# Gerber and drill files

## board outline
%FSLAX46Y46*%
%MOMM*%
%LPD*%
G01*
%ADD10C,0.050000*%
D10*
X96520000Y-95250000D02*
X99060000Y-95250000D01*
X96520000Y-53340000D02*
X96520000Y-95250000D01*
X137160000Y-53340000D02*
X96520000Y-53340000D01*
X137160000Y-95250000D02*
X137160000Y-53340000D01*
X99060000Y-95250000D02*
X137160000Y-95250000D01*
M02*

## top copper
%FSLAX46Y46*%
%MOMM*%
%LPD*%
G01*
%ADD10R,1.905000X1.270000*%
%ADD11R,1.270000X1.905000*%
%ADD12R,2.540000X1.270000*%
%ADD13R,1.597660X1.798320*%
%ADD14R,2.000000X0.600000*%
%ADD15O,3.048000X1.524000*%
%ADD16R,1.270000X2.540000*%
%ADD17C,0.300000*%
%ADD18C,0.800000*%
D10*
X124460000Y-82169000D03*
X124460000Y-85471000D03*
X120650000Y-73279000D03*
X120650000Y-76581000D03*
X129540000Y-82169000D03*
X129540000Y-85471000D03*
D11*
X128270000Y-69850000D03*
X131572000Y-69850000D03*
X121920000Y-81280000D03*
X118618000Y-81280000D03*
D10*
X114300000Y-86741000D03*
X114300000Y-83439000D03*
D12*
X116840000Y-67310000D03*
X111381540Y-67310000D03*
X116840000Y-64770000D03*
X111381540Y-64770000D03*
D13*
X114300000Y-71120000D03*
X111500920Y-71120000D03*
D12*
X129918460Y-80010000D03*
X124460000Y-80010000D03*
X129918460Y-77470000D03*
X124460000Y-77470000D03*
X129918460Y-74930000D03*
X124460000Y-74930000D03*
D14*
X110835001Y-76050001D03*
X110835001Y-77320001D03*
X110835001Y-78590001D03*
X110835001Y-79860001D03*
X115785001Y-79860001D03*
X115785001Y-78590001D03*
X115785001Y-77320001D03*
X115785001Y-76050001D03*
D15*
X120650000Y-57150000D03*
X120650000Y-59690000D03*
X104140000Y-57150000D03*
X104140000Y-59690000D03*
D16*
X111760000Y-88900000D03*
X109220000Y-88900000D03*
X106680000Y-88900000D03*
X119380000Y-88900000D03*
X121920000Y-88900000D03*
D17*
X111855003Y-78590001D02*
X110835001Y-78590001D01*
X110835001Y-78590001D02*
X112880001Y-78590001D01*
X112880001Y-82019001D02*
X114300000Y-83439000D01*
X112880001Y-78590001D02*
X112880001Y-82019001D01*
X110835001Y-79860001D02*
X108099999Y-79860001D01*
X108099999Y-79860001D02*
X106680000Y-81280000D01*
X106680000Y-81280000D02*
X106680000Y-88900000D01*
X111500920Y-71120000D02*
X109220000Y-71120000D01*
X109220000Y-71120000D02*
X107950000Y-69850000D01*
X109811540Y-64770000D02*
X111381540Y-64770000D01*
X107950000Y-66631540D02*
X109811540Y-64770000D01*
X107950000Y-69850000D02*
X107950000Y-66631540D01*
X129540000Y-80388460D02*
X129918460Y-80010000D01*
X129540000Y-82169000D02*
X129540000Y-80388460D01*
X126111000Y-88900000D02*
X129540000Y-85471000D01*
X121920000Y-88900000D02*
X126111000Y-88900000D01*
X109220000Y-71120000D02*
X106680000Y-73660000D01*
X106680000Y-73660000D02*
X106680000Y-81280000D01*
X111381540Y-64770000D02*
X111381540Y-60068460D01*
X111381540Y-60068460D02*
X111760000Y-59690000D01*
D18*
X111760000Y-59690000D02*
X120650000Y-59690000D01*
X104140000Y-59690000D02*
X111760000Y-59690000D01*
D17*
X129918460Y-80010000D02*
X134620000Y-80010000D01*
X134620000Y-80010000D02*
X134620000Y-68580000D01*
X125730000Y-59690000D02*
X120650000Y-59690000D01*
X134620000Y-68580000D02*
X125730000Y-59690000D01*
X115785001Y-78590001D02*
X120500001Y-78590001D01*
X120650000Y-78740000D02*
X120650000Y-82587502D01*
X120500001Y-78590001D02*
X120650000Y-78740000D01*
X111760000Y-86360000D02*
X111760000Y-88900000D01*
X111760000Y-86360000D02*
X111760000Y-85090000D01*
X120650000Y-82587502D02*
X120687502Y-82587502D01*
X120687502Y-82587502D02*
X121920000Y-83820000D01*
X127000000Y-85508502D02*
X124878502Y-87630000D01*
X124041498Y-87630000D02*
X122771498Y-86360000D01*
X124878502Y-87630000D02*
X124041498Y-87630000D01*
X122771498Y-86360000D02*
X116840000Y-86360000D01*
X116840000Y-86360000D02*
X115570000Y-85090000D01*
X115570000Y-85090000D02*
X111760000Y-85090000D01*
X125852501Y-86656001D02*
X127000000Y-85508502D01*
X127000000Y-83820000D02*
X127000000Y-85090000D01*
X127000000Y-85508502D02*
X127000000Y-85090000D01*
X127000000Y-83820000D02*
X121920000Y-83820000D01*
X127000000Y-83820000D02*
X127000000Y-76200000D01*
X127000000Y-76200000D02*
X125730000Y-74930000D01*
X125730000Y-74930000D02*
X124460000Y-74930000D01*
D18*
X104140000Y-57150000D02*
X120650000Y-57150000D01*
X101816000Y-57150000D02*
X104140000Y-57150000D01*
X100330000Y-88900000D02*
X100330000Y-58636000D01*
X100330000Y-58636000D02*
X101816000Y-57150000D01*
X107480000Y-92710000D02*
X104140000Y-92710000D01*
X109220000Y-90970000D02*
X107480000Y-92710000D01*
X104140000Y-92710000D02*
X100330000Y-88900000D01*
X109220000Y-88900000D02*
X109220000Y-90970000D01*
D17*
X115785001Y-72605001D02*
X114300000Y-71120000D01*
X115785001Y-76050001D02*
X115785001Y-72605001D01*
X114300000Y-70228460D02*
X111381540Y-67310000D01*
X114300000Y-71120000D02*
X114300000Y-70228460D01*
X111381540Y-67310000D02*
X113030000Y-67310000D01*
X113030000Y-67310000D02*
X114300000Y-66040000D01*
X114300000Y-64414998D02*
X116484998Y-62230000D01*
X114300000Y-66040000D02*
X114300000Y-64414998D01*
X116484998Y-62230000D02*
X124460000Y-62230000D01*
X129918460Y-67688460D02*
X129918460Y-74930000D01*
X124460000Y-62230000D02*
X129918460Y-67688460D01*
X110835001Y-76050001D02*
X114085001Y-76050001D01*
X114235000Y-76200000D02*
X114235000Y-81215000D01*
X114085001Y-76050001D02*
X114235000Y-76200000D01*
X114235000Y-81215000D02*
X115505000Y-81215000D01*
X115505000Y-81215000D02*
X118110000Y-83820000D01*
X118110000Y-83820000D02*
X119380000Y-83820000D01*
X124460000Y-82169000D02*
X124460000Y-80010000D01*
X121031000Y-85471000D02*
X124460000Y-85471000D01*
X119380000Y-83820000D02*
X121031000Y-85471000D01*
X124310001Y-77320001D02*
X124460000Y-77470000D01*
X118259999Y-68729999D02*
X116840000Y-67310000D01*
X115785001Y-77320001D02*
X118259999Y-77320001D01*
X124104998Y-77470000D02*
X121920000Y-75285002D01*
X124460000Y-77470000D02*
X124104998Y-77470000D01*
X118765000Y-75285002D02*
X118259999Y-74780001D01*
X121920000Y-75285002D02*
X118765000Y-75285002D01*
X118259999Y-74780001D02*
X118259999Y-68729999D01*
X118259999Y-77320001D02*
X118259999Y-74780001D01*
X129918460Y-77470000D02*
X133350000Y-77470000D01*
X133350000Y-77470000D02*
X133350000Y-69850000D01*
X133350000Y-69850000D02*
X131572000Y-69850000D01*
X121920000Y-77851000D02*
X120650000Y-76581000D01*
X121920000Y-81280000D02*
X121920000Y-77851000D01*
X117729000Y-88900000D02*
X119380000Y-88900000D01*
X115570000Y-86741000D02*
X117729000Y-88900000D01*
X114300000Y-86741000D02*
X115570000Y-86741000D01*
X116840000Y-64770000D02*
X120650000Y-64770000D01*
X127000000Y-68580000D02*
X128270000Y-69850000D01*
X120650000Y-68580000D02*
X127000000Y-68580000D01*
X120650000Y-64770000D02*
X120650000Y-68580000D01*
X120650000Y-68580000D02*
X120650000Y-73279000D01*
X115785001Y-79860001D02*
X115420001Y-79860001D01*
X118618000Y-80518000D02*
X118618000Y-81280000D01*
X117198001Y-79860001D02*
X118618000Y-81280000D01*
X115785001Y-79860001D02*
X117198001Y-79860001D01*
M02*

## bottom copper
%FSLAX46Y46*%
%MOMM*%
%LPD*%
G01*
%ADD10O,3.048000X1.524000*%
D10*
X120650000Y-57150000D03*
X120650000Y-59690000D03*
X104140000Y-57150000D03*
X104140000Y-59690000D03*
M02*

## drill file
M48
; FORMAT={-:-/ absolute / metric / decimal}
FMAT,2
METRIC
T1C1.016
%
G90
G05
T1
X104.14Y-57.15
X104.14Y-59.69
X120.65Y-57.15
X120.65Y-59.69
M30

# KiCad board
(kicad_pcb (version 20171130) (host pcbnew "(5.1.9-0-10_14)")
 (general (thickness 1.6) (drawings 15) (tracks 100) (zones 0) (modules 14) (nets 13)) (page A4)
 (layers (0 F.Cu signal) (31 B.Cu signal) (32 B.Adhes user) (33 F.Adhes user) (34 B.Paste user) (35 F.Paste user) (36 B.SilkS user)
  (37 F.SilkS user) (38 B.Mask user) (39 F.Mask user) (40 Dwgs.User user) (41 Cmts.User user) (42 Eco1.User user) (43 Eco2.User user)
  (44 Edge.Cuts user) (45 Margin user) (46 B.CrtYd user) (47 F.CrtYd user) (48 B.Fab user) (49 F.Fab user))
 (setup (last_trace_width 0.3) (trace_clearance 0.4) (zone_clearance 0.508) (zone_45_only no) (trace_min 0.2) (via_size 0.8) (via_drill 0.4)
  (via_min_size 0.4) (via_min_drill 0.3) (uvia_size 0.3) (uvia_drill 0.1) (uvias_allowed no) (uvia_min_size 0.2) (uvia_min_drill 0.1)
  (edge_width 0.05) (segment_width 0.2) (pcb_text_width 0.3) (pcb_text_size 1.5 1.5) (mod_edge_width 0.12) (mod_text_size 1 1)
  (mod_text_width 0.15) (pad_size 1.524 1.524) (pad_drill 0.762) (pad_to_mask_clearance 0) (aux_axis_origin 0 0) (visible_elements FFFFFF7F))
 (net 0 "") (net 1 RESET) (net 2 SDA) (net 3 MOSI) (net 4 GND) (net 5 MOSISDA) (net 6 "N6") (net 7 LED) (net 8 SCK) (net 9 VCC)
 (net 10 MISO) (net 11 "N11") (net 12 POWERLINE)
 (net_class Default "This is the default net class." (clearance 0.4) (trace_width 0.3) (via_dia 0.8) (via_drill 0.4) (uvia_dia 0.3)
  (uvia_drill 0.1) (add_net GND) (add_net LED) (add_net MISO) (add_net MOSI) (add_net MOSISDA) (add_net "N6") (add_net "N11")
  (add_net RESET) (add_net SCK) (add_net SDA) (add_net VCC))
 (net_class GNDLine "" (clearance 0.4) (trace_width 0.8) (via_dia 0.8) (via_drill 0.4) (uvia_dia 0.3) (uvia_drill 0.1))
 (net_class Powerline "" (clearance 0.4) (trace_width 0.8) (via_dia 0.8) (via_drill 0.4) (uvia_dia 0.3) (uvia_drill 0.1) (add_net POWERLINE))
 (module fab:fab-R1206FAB (layer F.Cu) (at 124.46 83.82 90)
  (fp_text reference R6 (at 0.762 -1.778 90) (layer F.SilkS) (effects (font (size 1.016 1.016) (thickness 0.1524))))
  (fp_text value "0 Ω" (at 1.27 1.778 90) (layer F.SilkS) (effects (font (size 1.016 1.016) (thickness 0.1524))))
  (pad 2 smd rect (at 1.651 0 90) (size 1.27 1.905) (layers F.Cu F.Paste F.Mask) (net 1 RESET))
  (pad 1 smd rect (at -1.651 0 90) (size 1.27 1.905) (layers F.Cu F.Paste F.Mask) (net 1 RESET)))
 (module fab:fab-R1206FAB (layer F.Cu) (at 120.65 74.93 90)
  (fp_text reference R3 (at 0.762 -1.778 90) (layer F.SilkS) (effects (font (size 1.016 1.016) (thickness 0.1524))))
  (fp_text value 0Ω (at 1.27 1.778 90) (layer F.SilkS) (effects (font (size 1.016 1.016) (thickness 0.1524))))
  (pad 2 smd rect (at 1.651 0 90) (size 1.27 1.905) (layers F.Cu F.Paste F.Mask) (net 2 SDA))
  (pad 1 smd rect (at -1.651 0 90) (size 1.27 1.905) (layers F.Cu F.Paste F.Mask) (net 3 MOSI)))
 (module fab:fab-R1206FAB (layer F.Cu) (at 129.54 83.82 90)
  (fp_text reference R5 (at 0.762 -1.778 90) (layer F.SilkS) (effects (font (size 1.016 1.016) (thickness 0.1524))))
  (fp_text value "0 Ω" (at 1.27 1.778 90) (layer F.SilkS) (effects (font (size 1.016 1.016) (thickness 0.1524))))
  (pad 2 smd rect (at 1.651 0 90) (size 1.27 1.905) (layers F.Cu F.Paste F.Mask) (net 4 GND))
  (pad 1 smd rect (at -1.651 0 90) (size 1.27 1.905) (layers F.Cu F.Paste F.Mask) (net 4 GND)))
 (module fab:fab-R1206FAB (layer F.Cu) (at 129.921 69.85 180)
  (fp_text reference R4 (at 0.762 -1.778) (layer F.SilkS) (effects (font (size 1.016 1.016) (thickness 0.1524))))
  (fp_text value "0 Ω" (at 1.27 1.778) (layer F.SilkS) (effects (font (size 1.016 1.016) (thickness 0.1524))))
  (pad 2 smd rect (at 1.651 0 180) (size 1.27 1.905) (layers F.Cu F.Paste F.Mask) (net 2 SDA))
  (pad 1 smd rect (at -1.651 0 180) (size 1.27 1.905) (layers F.Cu F.Paste F.Mask) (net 3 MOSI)))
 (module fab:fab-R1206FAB (layer F.Cu) (at 120.269 81.28)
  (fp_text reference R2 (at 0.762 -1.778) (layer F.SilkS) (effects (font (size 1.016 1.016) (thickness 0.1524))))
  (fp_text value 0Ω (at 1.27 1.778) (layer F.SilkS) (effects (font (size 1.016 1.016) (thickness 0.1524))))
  (pad 2 smd rect (at 1.651 0) (size 1.27 1.905) (layers F.Cu F.Paste F.Mask) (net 3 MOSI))
  (pad 1 smd rect (at -1.651 0) (size 1.27 1.905) (layers F.Cu F.Paste F.Mask) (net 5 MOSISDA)))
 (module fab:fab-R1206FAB (layer F.Cu) (at 114.3 85.09 270)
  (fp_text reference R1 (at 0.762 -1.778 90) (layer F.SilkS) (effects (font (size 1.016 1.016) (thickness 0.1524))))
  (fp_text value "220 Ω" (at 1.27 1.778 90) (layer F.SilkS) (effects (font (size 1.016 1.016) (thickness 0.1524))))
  (pad 2 smd rect (at 1.651 0 270) (size 1.27 1.905) (layers F.Cu F.Paste F.Mask) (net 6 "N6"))
  (pad 1 smd rect (at -1.651 0 270) (size 1.27 1.905) (layers F.Cu F.Paste F.Mask) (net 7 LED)))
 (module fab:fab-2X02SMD (layer F.Cu) (at 113.92154 66.04)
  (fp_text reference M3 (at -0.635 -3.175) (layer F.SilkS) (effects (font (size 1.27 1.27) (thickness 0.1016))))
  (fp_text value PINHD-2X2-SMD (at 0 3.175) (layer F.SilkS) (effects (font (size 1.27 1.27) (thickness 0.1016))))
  (pad 4 smd rect (at 2.91846 1.27) (size 2.54 1.27) (layers F.Cu F.Paste F.Mask) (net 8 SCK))
  (pad 3 smd rect (at -2.54 1.27) (size 2.54 1.27) (layers F.Cu F.Paste F.Mask) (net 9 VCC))
  (pad 2 smd rect (at 2.91846 -1.27) (size 2.54 1.27) (layers F.Cu F.Paste F.Mask) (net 2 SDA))
  (pad 1 smd rect (at -2.54 -1.27) (size 2.54 1.27) (layers F.Cu F.Paste F.Mask) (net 4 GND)))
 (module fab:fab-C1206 (layer F.Cu) (at 112.90046 71.12)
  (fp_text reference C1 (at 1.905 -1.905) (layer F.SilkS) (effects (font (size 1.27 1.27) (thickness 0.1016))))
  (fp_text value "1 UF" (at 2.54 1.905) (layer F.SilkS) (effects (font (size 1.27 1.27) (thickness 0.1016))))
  (pad 2 smd rect (at 1.39954 0) (size 1.59766 1.79832) (layers F.Cu F.Paste F.Mask) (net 9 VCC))
  (pad 1 smd rect (at -1.39954 0) (size 1.59766 1.79832) (layers F.Cu F.Paste F.Mask) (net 4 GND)))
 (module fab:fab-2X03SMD (layer F.Cu) (at 127 77.47)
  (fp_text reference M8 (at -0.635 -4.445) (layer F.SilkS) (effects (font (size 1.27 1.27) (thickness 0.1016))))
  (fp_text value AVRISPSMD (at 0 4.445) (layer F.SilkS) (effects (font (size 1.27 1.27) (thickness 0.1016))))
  (pad 6 smd rect (at 2.91846 2.54) (size 2.54 1.27) (layers F.Cu F.Paste F.Mask) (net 4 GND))
  (pad 5 smd rect (at -2.54 2.54) (size 2.54 1.27) (layers F.Cu F.Paste F.Mask) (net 1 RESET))
  (pad 4 smd rect (at 2.91846 0) (size 2.54 1.27) (layers F.Cu F.Paste F.Mask) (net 3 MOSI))
  (pad 3 smd rect (at -2.54 0) (size 2.54 1.27) (layers F.Cu F.Paste F.Mask) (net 8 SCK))
  (pad 2 smd rect (at 2.91846 -2.54) (size 2.54 1.27) (layers F.Cu F.Paste F.Mask) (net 9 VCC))
  (pad 1 smd rect (at -2.54 -2.54) (size 2.54 1.27) (layers F.Cu F.Paste F.Mask) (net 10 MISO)))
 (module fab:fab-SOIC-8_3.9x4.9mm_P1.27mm (layer F.Cu) (at 113.310001 77.955001)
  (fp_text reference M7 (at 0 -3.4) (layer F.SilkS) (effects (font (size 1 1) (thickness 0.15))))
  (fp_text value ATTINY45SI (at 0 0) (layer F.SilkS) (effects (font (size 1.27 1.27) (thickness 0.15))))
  (pad 1 smd rect (at -2.475 -1.905) (size 2 0.6) (layers F.Cu) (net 1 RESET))
  (pad 2 smd rect (at -2.475 -0.635) (size 2 0.6) (layers F.Cu) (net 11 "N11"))
  (pad 3 smd rect (at -2.475 0.635) (size 2 0.6) (layers F.Cu) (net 7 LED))
  (pad 4 smd rect (at -2.475 1.905) (size 2 0.6) (layers F.Cu) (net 4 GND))
  (pad 5 smd rect (at 2.475 1.905) (size 2 0.6) (layers F.Cu) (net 5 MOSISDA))
  (pad 6 smd rect (at 2.475 0.635) (size 2 0.6) (layers F.Cu) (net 10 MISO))
  (pad 7 smd rect (at 2.475 -0.635) (size 2 0.6) (layers F.Cu) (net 8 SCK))
  (pad 8 smd rect (at 2.475 -1.905) (size 2 0.6) (layers F.Cu) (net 9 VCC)))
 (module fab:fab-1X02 (layer F.Cu) (at 120.65 58.42 90)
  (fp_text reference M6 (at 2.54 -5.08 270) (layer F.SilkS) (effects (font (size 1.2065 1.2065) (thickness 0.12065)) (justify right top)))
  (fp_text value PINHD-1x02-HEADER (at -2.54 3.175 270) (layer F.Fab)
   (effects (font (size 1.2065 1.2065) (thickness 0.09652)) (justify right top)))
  (pad 2 thru_hole oval (at 1.27 0 180) (size 3.048 1.524) (drill 1.016) (layers *.Cu *.Mask) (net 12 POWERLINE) (solder_mask_margin 0.1016))
  (pad 1 thru_hole oval (at -1.27 0 180) (size 3.048 1.524) (drill 1.016) (layers *.Cu *.Mask) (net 4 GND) (solder_mask_margin 0.1016)))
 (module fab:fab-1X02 (layer F.Cu) (at 104.14 58.42 90)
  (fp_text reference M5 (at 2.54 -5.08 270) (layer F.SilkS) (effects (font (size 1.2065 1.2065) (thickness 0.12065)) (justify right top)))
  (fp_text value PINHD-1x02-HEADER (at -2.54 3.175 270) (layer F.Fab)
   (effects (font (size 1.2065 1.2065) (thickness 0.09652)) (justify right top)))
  (pad 2 thru_hole oval (at 1.27 0 180) (size 3.048 1.524) (drill 1.016) (layers *.Cu *.Mask) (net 12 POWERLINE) (solder_mask_margin 0.1016))
  (pad 1 thru_hole oval (at -1.27 0 180) (size 3.048 1.524) (drill 1.016) (layers *.Cu *.Mask) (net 4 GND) (solder_mask_margin 0.1016)))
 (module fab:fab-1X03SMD (layer F.Cu) (at 109.22 88.9 90)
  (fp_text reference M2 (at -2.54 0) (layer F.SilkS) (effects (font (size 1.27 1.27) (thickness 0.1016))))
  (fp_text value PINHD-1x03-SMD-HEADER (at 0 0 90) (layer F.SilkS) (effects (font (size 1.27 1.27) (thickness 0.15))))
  (pad 3 smd rect (at 0 2.54 90) (size 2.54 1.27) (layers F.Cu F.Paste F.Mask) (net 10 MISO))
  (pad 2 smd rect (at 0 0 90) (size 2.54 1.27) (layers F.Cu F.Paste F.Mask) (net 12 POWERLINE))
  (pad 1 smd rect (at 0 -2.54 90) (size 2.54 1.27) (layers F.Cu F.Paste F.Mask) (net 4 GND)))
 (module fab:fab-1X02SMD (layer F.Cu) (at 120.65 88.9 270)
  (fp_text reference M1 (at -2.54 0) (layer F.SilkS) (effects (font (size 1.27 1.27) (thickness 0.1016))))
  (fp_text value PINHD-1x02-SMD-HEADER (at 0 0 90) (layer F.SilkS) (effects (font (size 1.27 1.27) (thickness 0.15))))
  (pad 2 smd rect (at 0 1.27 270) (size 2.54 1.27) (layers F.Cu F.Paste F.Mask) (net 6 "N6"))
  (pad 1 smd rect (at 0 -1.27 270) (size 2.54 1.27) (layers F.Cu F.Paste F.Mask) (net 4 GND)))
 (gr_line (start 96.52 95.25) (end 99.06 95.25) (layer Edge.Cuts) (width 0.05))
 (gr_line (start 96.52 53.34) (end 96.52 95.25) (layer Edge.Cuts) (width 0.05))
 (gr_line (start 137.16 53.34) (end 96.52 53.34) (layer Edge.Cuts) (width 0.05))
 (gr_line (start 137.16 95.25) (end 137.16 53.34) (layer Edge.Cuts) (width 0.05))
 (gr_line (start 99.06 95.25) (end 137.16 95.25) (layer Edge.Cuts) (width 0.05))
 (segment (start 111.855003 78.590001) (end 110.835001 78.590001) (width 0.3) (layer F.Cu) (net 7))
 (segment (start 110.835001 78.590001) (end 112.880001 78.590001) (width 0.3) (layer F.Cu) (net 7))
 (segment (start 112.880001 82.019001) (end 114.3 83.439) (width 0.3) (layer F.Cu) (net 7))
 (segment (start 112.880001 78.590001) (end 112.880001 82.019001) (width 0.3) (layer F.Cu) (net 7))
 (segment (start 110.835001 79.860001) (end 108.099999 79.860001) (width 0.3) (layer F.Cu) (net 4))
 (segment (start 108.099999 79.860001) (end 106.68 81.28) (width 0.3) (layer F.Cu) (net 4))
 (segment (start 106.68 81.28) (end 106.68 88.9) (width 0.3) (layer F.Cu) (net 4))
 (segment (start 111.50092 71.12) (end 109.22 71.12) (width 0.3) (layer F.Cu) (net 4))
 (segment (start 109.22 71.12) (end 107.95 69.85) (width 0.3) (layer F.Cu) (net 4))
 (segment (start 109.81154 64.77) (end 111.38154 64.77) (width 0.3) (layer F.Cu) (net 4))
 (segment (start 107.95 66.63154) (end 109.81154 64.77) (width 0.3) (layer F.Cu) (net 4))
 (segment (start 107.95 69.85) (end 107.95 66.63154) (width 0.3) (layer F.Cu) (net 4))
 (segment (start 129.54 80.38846) (end 129.91846 80.01) (width 0.3) (layer F.Cu) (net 4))
 (segment (start 129.54 82.169) (end 129.54 80.38846) (width 0.3) (layer F.Cu) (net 4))
 (segment (start 126.111 88.9) (end 129.54 85.471) (width 0.3) (layer F.Cu) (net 4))
 (segment (start 121.92 88.9) (end 126.111 88.9) (width 0.3) (layer F.Cu) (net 4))
 (segment (start 109.22 71.12) (end 106.68 73.66) (width 0.3) (layer F.Cu) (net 4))
 (segment (start 106.68 73.66) (end 106.68 81.28) (width 0.3) (layer F.Cu) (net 4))
 (segment (start 111.38154 64.77) (end 111.38154 60.06846) (width 0.3) (layer F.Cu) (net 4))
 (segment (start 111.38154 60.06846) (end 111.76 59.69) (width 0.3) (layer F.Cu) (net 4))
 (segment (start 111.76 59.69) (end 120.65 59.69) (width 0.8) (layer F.Cu) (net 4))
 (segment (start 104.14 59.69) (end 111.76 59.69) (width 0.8) (layer F.Cu) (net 4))
 (segment (start 129.91846 80.01) (end 134.62 80.01) (width 0.3) (layer F.Cu) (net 4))
 (segment (start 134.62 80.01) (end 134.62 68.58) (width 0.3) (layer F.Cu) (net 4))
 (segment (start 125.73 59.69) (end 120.65 59.69) (width 0.3) (layer F.Cu) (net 4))
 (segment (start 134.62 68.58) (end 125.73 59.69) (width 0.3) (layer F.Cu) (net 4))
 (segment (start 115.785001 78.590001) (end 120.500001 78.590001) (width 0.3) (layer F.Cu) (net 10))
 (segment (start 120.65 78.74) (end 120.65 82.587502) (width 0.3) (layer F.Cu) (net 10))
 (segment (start 120.500001 78.590001) (end 120.65 78.74) (width 0.3) (layer F.Cu) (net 10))
 (segment (start 111.76 86.36) (end 111.76 88.9) (width 0.3) (layer F.Cu) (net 10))
 (segment (start 111.76 86.36) (end 111.76 85.09) (width 0.3) (layer F.Cu) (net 10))
 (segment (start 120.65 82.587502) (end 120.687502 82.587502) (width 0.3) (layer F.Cu) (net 10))
 (segment (start 120.687502 82.587502) (end 121.92 83.82) (width 0.3) (layer F.Cu) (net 10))
 (segment (start 127 85.508502) (end 124.878502 87.63) (width 0.3) (layer F.Cu) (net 10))
 (segment (start 124.041498 87.63) (end 122.771498 86.36) (width 0.3) (layer F.Cu) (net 10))
 (segment (start 124.878502 87.63) (end 124.041498 87.63) (width 0.3) (layer F.Cu) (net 10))
 (segment (start 122.771498 86.36) (end 116.84 86.36) (width 0.3) (layer F.Cu) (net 10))
 (segment (start 116.84 86.36) (end 115.57 85.09) (width 0.3) (layer F.Cu) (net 10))
 (segment (start 115.57 85.09) (end 111.76 85.09) (width 0.3) (layer F.Cu) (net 10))
 (segment (start 125.852501 86.656001) (end 127 85.508502) (width 0.3) (layer F.Cu) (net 10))
 (segment (start 127 83.82) (end 127 85.09) (width 0.3) (layer F.Cu) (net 10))
 (segment (start 127 85.508502) (end 127 85.09) (width 0.3) (layer F.Cu) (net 10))
 (segment (start 127 83.82) (end 121.92 83.82) (width 0.3) (layer F.Cu) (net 10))
 (segment (start 127 83.82) (end 127 76.2) (width 0.3) (layer F.Cu) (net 10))
 (segment (start 127 76.2) (end 125.73 74.93) (width 0.3) (layer F.Cu) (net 10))
 (segment (start 125.73 74.93) (end 124.46 74.93) (width 0.3) (layer F.Cu) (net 10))
 (segment (start 104.14 57.15) (end 120.65 57.15) (width 0.8) (layer F.Cu) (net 12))
 (segment (start 101.816 57.15) (end 104.14 57.15) (width 0.8) (layer F.Cu) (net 12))
 (segment (start 100.33 88.9) (end 100.33 58.636) (width 0.8) (layer F.Cu) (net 12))
 (segment (start 100.33 58.636) (end 101.816 57.15) (width 0.8) (layer F.Cu) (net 12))
 (segment (start 107.48 92.71) (end 104.14 92.71) (width 0.8) (layer F.Cu) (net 12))
 (segment (start 109.22 90.97) (end 107.48 92.71) (width 0.8) (layer F.Cu) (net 12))
 (segment (start 104.14 92.71) (end 100.33 88.9) (width 0.8) (layer F.Cu) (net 12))
 (segment (start 109.22 88.9) (end 109.22 90.97) (width 0.8) (layer F.Cu) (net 12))
 (segment (start 115.785001 72.605001) (end 114.3 71.12) (width 0.3) (layer F.Cu) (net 9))
 (segment (start 115.785001 76.050001) (end 115.785001 72.605001) (width 0.3) (layer F.Cu) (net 9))
 (segment (start 114.3 70.22846) (end 111.38154 67.31) (width 0.3) (layer F.Cu) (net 9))
 (segment (start 114.3 71.12) (end 114.3 70.22846) (width 0.3) (layer F.Cu) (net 9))
 (segment (start 111.38154 67.31) (end 113.03 67.31) (width 0.3) (layer F.Cu) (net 9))
 (segment (start 113.03 67.31) (end 114.3 66.04) (width 0.3) (layer F.Cu) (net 9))
 (segment (start 114.3 64.414998) (end 116.484998 62.23) (width 0.3) (layer F.Cu) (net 9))
 (segment (start 114.3 66.04) (end 114.3 64.414998) (width 0.3) (layer F.Cu) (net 9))
 (segment (start 116.484998 62.23) (end 124.46 62.23) (width 0.3) (layer F.Cu) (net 9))
 (segment (start 129.91846 67.68846) (end 129.91846 74.93) (width 0.3) (layer F.Cu) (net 9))
 (segment (start 124.46 62.23) (end 129.91846 67.68846) (width 0.3) (layer F.Cu) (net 9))
 (segment (start 110.835001 76.050001) (end 114.085001 76.050001) (width 0.3) (layer F.Cu) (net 1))
 (segment (start 114.235 76.2) (end 114.235 81.215) (width 0.3) (layer F.Cu) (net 1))
 (segment (start 114.085001 76.050001) (end 114.235 76.2) (width 0.3) (layer F.Cu) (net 1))
 (segment (start 114.235 81.215) (end 115.505 81.215) (width 0.3) (layer F.Cu) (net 1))
 (segment (start 115.505 81.215) (end 118.11 83.82) (width 0.3) (layer F.Cu) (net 1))
 (segment (start 118.11 83.82) (end 119.38 83.82) (width 0.3) (layer F.Cu) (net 1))
 (segment (start 124.46 82.169) (end 124.46 80.01) (width 0.3) (layer F.Cu) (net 1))
 (segment (start 121.031 85.471) (end 124.46 85.471) (width 0.3) (layer F.Cu) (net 1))
 (segment (start 119.38 83.82) (end 121.031 85.471) (width 0.3) (layer F.Cu) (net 1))
 (segment (start 124.310001 77.320001) (end 124.46 77.47) (width 0.3) (layer F.Cu) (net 8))
 (segment (start 118.259999 68.729999) (end 116.84 67.31) (width 0.3) (layer F.Cu) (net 8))
 (segment (start 115.785001 77.320001) (end 118.259999 77.320001) (width 0.3) (layer F.Cu) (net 8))
 (segment (start 124.104998 77.47) (end 121.92 75.285002) (width 0.3) (layer F.Cu) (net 8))
 (segment (start 124.46 77.47) (end 124.104998 77.47) (width 0.3) (layer F.Cu) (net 8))
 (segment (start 118.765 75.285002) (end 118.259999 74.780001) (width 0.3) (layer F.Cu) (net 8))
 (segment (start 121.92 75.285002) (end 118.765 75.285002) (width 0.3) (layer F.Cu) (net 8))
 (segment (start 118.259999 74.780001) (end 118.259999 68.729999) (width 0.3) (layer F.Cu) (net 8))
 (segment (start 118.259999 77.320001) (end 118.259999 74.780001) (width 0.3) (layer F.Cu) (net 8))
 (segment (start 129.91846 77.47) (end 133.35 77.47) (width 0.3) (layer F.Cu) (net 3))
 (segment (start 133.35 77.47) (end 133.35 69.85) (width 0.3) (layer F.Cu) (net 3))
 (segment (start 133.35 69.85) (end 131.572 69.85) (width 0.3) (layer F.Cu) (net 3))
 (segment (start 121.92 77.851) (end 120.65 76.581) (width 0.3) (layer F.Cu) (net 3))
 (segment (start 121.92 81.28) (end 121.92 77.851) (width 0.3) (layer F.Cu) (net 3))
 (segment (start 117.729 88.9) (end 119.38 88.9) (width 0.3) (layer F.Cu) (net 6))
 (segment (start 115.57 86.741) (end 117.729 88.9) (width 0.3) (layer F.Cu) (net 6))
 (segment (start 114.3 86.741) (end 115.57 86.741) (width 0.3) (layer F.Cu) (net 6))
 (segment (start 116.84 64.77) (end 120.65 64.77) (width 0.3) (layer F.Cu) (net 2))
 (segment (start 127 68.58) (end 128.27 69.85) (width 0.3) (layer F.Cu) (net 2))
 (segment (start 120.65 68.58) (end 127 68.58) (width 0.3) (layer F.Cu) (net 2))
 (segment (start 120.65 64.77) (end 120.65 68.58) (width 0.3) (layer F.Cu) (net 2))
 (segment (start 120.65 68.58) (end 120.65 73.279) (width 0.3) (layer F.Cu) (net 2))
 (segment (start 115.785001 79.860001) (end 115.420001 79.860001) (width 0.3) (layer F.Cu) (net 5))
 (segment (start 118.618 80.518) (end 118.618 81.28) (width 0.3) (layer F.Cu) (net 5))
 (segment (start 117.198001 79.860001) (end 118.618 81.28) (width 0.3) (layer F.Cu) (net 5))
 (segment (start 115.785001 79.860001) (end 117.198001 79.860001) (width 0.3) (layer F.Cu) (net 5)))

